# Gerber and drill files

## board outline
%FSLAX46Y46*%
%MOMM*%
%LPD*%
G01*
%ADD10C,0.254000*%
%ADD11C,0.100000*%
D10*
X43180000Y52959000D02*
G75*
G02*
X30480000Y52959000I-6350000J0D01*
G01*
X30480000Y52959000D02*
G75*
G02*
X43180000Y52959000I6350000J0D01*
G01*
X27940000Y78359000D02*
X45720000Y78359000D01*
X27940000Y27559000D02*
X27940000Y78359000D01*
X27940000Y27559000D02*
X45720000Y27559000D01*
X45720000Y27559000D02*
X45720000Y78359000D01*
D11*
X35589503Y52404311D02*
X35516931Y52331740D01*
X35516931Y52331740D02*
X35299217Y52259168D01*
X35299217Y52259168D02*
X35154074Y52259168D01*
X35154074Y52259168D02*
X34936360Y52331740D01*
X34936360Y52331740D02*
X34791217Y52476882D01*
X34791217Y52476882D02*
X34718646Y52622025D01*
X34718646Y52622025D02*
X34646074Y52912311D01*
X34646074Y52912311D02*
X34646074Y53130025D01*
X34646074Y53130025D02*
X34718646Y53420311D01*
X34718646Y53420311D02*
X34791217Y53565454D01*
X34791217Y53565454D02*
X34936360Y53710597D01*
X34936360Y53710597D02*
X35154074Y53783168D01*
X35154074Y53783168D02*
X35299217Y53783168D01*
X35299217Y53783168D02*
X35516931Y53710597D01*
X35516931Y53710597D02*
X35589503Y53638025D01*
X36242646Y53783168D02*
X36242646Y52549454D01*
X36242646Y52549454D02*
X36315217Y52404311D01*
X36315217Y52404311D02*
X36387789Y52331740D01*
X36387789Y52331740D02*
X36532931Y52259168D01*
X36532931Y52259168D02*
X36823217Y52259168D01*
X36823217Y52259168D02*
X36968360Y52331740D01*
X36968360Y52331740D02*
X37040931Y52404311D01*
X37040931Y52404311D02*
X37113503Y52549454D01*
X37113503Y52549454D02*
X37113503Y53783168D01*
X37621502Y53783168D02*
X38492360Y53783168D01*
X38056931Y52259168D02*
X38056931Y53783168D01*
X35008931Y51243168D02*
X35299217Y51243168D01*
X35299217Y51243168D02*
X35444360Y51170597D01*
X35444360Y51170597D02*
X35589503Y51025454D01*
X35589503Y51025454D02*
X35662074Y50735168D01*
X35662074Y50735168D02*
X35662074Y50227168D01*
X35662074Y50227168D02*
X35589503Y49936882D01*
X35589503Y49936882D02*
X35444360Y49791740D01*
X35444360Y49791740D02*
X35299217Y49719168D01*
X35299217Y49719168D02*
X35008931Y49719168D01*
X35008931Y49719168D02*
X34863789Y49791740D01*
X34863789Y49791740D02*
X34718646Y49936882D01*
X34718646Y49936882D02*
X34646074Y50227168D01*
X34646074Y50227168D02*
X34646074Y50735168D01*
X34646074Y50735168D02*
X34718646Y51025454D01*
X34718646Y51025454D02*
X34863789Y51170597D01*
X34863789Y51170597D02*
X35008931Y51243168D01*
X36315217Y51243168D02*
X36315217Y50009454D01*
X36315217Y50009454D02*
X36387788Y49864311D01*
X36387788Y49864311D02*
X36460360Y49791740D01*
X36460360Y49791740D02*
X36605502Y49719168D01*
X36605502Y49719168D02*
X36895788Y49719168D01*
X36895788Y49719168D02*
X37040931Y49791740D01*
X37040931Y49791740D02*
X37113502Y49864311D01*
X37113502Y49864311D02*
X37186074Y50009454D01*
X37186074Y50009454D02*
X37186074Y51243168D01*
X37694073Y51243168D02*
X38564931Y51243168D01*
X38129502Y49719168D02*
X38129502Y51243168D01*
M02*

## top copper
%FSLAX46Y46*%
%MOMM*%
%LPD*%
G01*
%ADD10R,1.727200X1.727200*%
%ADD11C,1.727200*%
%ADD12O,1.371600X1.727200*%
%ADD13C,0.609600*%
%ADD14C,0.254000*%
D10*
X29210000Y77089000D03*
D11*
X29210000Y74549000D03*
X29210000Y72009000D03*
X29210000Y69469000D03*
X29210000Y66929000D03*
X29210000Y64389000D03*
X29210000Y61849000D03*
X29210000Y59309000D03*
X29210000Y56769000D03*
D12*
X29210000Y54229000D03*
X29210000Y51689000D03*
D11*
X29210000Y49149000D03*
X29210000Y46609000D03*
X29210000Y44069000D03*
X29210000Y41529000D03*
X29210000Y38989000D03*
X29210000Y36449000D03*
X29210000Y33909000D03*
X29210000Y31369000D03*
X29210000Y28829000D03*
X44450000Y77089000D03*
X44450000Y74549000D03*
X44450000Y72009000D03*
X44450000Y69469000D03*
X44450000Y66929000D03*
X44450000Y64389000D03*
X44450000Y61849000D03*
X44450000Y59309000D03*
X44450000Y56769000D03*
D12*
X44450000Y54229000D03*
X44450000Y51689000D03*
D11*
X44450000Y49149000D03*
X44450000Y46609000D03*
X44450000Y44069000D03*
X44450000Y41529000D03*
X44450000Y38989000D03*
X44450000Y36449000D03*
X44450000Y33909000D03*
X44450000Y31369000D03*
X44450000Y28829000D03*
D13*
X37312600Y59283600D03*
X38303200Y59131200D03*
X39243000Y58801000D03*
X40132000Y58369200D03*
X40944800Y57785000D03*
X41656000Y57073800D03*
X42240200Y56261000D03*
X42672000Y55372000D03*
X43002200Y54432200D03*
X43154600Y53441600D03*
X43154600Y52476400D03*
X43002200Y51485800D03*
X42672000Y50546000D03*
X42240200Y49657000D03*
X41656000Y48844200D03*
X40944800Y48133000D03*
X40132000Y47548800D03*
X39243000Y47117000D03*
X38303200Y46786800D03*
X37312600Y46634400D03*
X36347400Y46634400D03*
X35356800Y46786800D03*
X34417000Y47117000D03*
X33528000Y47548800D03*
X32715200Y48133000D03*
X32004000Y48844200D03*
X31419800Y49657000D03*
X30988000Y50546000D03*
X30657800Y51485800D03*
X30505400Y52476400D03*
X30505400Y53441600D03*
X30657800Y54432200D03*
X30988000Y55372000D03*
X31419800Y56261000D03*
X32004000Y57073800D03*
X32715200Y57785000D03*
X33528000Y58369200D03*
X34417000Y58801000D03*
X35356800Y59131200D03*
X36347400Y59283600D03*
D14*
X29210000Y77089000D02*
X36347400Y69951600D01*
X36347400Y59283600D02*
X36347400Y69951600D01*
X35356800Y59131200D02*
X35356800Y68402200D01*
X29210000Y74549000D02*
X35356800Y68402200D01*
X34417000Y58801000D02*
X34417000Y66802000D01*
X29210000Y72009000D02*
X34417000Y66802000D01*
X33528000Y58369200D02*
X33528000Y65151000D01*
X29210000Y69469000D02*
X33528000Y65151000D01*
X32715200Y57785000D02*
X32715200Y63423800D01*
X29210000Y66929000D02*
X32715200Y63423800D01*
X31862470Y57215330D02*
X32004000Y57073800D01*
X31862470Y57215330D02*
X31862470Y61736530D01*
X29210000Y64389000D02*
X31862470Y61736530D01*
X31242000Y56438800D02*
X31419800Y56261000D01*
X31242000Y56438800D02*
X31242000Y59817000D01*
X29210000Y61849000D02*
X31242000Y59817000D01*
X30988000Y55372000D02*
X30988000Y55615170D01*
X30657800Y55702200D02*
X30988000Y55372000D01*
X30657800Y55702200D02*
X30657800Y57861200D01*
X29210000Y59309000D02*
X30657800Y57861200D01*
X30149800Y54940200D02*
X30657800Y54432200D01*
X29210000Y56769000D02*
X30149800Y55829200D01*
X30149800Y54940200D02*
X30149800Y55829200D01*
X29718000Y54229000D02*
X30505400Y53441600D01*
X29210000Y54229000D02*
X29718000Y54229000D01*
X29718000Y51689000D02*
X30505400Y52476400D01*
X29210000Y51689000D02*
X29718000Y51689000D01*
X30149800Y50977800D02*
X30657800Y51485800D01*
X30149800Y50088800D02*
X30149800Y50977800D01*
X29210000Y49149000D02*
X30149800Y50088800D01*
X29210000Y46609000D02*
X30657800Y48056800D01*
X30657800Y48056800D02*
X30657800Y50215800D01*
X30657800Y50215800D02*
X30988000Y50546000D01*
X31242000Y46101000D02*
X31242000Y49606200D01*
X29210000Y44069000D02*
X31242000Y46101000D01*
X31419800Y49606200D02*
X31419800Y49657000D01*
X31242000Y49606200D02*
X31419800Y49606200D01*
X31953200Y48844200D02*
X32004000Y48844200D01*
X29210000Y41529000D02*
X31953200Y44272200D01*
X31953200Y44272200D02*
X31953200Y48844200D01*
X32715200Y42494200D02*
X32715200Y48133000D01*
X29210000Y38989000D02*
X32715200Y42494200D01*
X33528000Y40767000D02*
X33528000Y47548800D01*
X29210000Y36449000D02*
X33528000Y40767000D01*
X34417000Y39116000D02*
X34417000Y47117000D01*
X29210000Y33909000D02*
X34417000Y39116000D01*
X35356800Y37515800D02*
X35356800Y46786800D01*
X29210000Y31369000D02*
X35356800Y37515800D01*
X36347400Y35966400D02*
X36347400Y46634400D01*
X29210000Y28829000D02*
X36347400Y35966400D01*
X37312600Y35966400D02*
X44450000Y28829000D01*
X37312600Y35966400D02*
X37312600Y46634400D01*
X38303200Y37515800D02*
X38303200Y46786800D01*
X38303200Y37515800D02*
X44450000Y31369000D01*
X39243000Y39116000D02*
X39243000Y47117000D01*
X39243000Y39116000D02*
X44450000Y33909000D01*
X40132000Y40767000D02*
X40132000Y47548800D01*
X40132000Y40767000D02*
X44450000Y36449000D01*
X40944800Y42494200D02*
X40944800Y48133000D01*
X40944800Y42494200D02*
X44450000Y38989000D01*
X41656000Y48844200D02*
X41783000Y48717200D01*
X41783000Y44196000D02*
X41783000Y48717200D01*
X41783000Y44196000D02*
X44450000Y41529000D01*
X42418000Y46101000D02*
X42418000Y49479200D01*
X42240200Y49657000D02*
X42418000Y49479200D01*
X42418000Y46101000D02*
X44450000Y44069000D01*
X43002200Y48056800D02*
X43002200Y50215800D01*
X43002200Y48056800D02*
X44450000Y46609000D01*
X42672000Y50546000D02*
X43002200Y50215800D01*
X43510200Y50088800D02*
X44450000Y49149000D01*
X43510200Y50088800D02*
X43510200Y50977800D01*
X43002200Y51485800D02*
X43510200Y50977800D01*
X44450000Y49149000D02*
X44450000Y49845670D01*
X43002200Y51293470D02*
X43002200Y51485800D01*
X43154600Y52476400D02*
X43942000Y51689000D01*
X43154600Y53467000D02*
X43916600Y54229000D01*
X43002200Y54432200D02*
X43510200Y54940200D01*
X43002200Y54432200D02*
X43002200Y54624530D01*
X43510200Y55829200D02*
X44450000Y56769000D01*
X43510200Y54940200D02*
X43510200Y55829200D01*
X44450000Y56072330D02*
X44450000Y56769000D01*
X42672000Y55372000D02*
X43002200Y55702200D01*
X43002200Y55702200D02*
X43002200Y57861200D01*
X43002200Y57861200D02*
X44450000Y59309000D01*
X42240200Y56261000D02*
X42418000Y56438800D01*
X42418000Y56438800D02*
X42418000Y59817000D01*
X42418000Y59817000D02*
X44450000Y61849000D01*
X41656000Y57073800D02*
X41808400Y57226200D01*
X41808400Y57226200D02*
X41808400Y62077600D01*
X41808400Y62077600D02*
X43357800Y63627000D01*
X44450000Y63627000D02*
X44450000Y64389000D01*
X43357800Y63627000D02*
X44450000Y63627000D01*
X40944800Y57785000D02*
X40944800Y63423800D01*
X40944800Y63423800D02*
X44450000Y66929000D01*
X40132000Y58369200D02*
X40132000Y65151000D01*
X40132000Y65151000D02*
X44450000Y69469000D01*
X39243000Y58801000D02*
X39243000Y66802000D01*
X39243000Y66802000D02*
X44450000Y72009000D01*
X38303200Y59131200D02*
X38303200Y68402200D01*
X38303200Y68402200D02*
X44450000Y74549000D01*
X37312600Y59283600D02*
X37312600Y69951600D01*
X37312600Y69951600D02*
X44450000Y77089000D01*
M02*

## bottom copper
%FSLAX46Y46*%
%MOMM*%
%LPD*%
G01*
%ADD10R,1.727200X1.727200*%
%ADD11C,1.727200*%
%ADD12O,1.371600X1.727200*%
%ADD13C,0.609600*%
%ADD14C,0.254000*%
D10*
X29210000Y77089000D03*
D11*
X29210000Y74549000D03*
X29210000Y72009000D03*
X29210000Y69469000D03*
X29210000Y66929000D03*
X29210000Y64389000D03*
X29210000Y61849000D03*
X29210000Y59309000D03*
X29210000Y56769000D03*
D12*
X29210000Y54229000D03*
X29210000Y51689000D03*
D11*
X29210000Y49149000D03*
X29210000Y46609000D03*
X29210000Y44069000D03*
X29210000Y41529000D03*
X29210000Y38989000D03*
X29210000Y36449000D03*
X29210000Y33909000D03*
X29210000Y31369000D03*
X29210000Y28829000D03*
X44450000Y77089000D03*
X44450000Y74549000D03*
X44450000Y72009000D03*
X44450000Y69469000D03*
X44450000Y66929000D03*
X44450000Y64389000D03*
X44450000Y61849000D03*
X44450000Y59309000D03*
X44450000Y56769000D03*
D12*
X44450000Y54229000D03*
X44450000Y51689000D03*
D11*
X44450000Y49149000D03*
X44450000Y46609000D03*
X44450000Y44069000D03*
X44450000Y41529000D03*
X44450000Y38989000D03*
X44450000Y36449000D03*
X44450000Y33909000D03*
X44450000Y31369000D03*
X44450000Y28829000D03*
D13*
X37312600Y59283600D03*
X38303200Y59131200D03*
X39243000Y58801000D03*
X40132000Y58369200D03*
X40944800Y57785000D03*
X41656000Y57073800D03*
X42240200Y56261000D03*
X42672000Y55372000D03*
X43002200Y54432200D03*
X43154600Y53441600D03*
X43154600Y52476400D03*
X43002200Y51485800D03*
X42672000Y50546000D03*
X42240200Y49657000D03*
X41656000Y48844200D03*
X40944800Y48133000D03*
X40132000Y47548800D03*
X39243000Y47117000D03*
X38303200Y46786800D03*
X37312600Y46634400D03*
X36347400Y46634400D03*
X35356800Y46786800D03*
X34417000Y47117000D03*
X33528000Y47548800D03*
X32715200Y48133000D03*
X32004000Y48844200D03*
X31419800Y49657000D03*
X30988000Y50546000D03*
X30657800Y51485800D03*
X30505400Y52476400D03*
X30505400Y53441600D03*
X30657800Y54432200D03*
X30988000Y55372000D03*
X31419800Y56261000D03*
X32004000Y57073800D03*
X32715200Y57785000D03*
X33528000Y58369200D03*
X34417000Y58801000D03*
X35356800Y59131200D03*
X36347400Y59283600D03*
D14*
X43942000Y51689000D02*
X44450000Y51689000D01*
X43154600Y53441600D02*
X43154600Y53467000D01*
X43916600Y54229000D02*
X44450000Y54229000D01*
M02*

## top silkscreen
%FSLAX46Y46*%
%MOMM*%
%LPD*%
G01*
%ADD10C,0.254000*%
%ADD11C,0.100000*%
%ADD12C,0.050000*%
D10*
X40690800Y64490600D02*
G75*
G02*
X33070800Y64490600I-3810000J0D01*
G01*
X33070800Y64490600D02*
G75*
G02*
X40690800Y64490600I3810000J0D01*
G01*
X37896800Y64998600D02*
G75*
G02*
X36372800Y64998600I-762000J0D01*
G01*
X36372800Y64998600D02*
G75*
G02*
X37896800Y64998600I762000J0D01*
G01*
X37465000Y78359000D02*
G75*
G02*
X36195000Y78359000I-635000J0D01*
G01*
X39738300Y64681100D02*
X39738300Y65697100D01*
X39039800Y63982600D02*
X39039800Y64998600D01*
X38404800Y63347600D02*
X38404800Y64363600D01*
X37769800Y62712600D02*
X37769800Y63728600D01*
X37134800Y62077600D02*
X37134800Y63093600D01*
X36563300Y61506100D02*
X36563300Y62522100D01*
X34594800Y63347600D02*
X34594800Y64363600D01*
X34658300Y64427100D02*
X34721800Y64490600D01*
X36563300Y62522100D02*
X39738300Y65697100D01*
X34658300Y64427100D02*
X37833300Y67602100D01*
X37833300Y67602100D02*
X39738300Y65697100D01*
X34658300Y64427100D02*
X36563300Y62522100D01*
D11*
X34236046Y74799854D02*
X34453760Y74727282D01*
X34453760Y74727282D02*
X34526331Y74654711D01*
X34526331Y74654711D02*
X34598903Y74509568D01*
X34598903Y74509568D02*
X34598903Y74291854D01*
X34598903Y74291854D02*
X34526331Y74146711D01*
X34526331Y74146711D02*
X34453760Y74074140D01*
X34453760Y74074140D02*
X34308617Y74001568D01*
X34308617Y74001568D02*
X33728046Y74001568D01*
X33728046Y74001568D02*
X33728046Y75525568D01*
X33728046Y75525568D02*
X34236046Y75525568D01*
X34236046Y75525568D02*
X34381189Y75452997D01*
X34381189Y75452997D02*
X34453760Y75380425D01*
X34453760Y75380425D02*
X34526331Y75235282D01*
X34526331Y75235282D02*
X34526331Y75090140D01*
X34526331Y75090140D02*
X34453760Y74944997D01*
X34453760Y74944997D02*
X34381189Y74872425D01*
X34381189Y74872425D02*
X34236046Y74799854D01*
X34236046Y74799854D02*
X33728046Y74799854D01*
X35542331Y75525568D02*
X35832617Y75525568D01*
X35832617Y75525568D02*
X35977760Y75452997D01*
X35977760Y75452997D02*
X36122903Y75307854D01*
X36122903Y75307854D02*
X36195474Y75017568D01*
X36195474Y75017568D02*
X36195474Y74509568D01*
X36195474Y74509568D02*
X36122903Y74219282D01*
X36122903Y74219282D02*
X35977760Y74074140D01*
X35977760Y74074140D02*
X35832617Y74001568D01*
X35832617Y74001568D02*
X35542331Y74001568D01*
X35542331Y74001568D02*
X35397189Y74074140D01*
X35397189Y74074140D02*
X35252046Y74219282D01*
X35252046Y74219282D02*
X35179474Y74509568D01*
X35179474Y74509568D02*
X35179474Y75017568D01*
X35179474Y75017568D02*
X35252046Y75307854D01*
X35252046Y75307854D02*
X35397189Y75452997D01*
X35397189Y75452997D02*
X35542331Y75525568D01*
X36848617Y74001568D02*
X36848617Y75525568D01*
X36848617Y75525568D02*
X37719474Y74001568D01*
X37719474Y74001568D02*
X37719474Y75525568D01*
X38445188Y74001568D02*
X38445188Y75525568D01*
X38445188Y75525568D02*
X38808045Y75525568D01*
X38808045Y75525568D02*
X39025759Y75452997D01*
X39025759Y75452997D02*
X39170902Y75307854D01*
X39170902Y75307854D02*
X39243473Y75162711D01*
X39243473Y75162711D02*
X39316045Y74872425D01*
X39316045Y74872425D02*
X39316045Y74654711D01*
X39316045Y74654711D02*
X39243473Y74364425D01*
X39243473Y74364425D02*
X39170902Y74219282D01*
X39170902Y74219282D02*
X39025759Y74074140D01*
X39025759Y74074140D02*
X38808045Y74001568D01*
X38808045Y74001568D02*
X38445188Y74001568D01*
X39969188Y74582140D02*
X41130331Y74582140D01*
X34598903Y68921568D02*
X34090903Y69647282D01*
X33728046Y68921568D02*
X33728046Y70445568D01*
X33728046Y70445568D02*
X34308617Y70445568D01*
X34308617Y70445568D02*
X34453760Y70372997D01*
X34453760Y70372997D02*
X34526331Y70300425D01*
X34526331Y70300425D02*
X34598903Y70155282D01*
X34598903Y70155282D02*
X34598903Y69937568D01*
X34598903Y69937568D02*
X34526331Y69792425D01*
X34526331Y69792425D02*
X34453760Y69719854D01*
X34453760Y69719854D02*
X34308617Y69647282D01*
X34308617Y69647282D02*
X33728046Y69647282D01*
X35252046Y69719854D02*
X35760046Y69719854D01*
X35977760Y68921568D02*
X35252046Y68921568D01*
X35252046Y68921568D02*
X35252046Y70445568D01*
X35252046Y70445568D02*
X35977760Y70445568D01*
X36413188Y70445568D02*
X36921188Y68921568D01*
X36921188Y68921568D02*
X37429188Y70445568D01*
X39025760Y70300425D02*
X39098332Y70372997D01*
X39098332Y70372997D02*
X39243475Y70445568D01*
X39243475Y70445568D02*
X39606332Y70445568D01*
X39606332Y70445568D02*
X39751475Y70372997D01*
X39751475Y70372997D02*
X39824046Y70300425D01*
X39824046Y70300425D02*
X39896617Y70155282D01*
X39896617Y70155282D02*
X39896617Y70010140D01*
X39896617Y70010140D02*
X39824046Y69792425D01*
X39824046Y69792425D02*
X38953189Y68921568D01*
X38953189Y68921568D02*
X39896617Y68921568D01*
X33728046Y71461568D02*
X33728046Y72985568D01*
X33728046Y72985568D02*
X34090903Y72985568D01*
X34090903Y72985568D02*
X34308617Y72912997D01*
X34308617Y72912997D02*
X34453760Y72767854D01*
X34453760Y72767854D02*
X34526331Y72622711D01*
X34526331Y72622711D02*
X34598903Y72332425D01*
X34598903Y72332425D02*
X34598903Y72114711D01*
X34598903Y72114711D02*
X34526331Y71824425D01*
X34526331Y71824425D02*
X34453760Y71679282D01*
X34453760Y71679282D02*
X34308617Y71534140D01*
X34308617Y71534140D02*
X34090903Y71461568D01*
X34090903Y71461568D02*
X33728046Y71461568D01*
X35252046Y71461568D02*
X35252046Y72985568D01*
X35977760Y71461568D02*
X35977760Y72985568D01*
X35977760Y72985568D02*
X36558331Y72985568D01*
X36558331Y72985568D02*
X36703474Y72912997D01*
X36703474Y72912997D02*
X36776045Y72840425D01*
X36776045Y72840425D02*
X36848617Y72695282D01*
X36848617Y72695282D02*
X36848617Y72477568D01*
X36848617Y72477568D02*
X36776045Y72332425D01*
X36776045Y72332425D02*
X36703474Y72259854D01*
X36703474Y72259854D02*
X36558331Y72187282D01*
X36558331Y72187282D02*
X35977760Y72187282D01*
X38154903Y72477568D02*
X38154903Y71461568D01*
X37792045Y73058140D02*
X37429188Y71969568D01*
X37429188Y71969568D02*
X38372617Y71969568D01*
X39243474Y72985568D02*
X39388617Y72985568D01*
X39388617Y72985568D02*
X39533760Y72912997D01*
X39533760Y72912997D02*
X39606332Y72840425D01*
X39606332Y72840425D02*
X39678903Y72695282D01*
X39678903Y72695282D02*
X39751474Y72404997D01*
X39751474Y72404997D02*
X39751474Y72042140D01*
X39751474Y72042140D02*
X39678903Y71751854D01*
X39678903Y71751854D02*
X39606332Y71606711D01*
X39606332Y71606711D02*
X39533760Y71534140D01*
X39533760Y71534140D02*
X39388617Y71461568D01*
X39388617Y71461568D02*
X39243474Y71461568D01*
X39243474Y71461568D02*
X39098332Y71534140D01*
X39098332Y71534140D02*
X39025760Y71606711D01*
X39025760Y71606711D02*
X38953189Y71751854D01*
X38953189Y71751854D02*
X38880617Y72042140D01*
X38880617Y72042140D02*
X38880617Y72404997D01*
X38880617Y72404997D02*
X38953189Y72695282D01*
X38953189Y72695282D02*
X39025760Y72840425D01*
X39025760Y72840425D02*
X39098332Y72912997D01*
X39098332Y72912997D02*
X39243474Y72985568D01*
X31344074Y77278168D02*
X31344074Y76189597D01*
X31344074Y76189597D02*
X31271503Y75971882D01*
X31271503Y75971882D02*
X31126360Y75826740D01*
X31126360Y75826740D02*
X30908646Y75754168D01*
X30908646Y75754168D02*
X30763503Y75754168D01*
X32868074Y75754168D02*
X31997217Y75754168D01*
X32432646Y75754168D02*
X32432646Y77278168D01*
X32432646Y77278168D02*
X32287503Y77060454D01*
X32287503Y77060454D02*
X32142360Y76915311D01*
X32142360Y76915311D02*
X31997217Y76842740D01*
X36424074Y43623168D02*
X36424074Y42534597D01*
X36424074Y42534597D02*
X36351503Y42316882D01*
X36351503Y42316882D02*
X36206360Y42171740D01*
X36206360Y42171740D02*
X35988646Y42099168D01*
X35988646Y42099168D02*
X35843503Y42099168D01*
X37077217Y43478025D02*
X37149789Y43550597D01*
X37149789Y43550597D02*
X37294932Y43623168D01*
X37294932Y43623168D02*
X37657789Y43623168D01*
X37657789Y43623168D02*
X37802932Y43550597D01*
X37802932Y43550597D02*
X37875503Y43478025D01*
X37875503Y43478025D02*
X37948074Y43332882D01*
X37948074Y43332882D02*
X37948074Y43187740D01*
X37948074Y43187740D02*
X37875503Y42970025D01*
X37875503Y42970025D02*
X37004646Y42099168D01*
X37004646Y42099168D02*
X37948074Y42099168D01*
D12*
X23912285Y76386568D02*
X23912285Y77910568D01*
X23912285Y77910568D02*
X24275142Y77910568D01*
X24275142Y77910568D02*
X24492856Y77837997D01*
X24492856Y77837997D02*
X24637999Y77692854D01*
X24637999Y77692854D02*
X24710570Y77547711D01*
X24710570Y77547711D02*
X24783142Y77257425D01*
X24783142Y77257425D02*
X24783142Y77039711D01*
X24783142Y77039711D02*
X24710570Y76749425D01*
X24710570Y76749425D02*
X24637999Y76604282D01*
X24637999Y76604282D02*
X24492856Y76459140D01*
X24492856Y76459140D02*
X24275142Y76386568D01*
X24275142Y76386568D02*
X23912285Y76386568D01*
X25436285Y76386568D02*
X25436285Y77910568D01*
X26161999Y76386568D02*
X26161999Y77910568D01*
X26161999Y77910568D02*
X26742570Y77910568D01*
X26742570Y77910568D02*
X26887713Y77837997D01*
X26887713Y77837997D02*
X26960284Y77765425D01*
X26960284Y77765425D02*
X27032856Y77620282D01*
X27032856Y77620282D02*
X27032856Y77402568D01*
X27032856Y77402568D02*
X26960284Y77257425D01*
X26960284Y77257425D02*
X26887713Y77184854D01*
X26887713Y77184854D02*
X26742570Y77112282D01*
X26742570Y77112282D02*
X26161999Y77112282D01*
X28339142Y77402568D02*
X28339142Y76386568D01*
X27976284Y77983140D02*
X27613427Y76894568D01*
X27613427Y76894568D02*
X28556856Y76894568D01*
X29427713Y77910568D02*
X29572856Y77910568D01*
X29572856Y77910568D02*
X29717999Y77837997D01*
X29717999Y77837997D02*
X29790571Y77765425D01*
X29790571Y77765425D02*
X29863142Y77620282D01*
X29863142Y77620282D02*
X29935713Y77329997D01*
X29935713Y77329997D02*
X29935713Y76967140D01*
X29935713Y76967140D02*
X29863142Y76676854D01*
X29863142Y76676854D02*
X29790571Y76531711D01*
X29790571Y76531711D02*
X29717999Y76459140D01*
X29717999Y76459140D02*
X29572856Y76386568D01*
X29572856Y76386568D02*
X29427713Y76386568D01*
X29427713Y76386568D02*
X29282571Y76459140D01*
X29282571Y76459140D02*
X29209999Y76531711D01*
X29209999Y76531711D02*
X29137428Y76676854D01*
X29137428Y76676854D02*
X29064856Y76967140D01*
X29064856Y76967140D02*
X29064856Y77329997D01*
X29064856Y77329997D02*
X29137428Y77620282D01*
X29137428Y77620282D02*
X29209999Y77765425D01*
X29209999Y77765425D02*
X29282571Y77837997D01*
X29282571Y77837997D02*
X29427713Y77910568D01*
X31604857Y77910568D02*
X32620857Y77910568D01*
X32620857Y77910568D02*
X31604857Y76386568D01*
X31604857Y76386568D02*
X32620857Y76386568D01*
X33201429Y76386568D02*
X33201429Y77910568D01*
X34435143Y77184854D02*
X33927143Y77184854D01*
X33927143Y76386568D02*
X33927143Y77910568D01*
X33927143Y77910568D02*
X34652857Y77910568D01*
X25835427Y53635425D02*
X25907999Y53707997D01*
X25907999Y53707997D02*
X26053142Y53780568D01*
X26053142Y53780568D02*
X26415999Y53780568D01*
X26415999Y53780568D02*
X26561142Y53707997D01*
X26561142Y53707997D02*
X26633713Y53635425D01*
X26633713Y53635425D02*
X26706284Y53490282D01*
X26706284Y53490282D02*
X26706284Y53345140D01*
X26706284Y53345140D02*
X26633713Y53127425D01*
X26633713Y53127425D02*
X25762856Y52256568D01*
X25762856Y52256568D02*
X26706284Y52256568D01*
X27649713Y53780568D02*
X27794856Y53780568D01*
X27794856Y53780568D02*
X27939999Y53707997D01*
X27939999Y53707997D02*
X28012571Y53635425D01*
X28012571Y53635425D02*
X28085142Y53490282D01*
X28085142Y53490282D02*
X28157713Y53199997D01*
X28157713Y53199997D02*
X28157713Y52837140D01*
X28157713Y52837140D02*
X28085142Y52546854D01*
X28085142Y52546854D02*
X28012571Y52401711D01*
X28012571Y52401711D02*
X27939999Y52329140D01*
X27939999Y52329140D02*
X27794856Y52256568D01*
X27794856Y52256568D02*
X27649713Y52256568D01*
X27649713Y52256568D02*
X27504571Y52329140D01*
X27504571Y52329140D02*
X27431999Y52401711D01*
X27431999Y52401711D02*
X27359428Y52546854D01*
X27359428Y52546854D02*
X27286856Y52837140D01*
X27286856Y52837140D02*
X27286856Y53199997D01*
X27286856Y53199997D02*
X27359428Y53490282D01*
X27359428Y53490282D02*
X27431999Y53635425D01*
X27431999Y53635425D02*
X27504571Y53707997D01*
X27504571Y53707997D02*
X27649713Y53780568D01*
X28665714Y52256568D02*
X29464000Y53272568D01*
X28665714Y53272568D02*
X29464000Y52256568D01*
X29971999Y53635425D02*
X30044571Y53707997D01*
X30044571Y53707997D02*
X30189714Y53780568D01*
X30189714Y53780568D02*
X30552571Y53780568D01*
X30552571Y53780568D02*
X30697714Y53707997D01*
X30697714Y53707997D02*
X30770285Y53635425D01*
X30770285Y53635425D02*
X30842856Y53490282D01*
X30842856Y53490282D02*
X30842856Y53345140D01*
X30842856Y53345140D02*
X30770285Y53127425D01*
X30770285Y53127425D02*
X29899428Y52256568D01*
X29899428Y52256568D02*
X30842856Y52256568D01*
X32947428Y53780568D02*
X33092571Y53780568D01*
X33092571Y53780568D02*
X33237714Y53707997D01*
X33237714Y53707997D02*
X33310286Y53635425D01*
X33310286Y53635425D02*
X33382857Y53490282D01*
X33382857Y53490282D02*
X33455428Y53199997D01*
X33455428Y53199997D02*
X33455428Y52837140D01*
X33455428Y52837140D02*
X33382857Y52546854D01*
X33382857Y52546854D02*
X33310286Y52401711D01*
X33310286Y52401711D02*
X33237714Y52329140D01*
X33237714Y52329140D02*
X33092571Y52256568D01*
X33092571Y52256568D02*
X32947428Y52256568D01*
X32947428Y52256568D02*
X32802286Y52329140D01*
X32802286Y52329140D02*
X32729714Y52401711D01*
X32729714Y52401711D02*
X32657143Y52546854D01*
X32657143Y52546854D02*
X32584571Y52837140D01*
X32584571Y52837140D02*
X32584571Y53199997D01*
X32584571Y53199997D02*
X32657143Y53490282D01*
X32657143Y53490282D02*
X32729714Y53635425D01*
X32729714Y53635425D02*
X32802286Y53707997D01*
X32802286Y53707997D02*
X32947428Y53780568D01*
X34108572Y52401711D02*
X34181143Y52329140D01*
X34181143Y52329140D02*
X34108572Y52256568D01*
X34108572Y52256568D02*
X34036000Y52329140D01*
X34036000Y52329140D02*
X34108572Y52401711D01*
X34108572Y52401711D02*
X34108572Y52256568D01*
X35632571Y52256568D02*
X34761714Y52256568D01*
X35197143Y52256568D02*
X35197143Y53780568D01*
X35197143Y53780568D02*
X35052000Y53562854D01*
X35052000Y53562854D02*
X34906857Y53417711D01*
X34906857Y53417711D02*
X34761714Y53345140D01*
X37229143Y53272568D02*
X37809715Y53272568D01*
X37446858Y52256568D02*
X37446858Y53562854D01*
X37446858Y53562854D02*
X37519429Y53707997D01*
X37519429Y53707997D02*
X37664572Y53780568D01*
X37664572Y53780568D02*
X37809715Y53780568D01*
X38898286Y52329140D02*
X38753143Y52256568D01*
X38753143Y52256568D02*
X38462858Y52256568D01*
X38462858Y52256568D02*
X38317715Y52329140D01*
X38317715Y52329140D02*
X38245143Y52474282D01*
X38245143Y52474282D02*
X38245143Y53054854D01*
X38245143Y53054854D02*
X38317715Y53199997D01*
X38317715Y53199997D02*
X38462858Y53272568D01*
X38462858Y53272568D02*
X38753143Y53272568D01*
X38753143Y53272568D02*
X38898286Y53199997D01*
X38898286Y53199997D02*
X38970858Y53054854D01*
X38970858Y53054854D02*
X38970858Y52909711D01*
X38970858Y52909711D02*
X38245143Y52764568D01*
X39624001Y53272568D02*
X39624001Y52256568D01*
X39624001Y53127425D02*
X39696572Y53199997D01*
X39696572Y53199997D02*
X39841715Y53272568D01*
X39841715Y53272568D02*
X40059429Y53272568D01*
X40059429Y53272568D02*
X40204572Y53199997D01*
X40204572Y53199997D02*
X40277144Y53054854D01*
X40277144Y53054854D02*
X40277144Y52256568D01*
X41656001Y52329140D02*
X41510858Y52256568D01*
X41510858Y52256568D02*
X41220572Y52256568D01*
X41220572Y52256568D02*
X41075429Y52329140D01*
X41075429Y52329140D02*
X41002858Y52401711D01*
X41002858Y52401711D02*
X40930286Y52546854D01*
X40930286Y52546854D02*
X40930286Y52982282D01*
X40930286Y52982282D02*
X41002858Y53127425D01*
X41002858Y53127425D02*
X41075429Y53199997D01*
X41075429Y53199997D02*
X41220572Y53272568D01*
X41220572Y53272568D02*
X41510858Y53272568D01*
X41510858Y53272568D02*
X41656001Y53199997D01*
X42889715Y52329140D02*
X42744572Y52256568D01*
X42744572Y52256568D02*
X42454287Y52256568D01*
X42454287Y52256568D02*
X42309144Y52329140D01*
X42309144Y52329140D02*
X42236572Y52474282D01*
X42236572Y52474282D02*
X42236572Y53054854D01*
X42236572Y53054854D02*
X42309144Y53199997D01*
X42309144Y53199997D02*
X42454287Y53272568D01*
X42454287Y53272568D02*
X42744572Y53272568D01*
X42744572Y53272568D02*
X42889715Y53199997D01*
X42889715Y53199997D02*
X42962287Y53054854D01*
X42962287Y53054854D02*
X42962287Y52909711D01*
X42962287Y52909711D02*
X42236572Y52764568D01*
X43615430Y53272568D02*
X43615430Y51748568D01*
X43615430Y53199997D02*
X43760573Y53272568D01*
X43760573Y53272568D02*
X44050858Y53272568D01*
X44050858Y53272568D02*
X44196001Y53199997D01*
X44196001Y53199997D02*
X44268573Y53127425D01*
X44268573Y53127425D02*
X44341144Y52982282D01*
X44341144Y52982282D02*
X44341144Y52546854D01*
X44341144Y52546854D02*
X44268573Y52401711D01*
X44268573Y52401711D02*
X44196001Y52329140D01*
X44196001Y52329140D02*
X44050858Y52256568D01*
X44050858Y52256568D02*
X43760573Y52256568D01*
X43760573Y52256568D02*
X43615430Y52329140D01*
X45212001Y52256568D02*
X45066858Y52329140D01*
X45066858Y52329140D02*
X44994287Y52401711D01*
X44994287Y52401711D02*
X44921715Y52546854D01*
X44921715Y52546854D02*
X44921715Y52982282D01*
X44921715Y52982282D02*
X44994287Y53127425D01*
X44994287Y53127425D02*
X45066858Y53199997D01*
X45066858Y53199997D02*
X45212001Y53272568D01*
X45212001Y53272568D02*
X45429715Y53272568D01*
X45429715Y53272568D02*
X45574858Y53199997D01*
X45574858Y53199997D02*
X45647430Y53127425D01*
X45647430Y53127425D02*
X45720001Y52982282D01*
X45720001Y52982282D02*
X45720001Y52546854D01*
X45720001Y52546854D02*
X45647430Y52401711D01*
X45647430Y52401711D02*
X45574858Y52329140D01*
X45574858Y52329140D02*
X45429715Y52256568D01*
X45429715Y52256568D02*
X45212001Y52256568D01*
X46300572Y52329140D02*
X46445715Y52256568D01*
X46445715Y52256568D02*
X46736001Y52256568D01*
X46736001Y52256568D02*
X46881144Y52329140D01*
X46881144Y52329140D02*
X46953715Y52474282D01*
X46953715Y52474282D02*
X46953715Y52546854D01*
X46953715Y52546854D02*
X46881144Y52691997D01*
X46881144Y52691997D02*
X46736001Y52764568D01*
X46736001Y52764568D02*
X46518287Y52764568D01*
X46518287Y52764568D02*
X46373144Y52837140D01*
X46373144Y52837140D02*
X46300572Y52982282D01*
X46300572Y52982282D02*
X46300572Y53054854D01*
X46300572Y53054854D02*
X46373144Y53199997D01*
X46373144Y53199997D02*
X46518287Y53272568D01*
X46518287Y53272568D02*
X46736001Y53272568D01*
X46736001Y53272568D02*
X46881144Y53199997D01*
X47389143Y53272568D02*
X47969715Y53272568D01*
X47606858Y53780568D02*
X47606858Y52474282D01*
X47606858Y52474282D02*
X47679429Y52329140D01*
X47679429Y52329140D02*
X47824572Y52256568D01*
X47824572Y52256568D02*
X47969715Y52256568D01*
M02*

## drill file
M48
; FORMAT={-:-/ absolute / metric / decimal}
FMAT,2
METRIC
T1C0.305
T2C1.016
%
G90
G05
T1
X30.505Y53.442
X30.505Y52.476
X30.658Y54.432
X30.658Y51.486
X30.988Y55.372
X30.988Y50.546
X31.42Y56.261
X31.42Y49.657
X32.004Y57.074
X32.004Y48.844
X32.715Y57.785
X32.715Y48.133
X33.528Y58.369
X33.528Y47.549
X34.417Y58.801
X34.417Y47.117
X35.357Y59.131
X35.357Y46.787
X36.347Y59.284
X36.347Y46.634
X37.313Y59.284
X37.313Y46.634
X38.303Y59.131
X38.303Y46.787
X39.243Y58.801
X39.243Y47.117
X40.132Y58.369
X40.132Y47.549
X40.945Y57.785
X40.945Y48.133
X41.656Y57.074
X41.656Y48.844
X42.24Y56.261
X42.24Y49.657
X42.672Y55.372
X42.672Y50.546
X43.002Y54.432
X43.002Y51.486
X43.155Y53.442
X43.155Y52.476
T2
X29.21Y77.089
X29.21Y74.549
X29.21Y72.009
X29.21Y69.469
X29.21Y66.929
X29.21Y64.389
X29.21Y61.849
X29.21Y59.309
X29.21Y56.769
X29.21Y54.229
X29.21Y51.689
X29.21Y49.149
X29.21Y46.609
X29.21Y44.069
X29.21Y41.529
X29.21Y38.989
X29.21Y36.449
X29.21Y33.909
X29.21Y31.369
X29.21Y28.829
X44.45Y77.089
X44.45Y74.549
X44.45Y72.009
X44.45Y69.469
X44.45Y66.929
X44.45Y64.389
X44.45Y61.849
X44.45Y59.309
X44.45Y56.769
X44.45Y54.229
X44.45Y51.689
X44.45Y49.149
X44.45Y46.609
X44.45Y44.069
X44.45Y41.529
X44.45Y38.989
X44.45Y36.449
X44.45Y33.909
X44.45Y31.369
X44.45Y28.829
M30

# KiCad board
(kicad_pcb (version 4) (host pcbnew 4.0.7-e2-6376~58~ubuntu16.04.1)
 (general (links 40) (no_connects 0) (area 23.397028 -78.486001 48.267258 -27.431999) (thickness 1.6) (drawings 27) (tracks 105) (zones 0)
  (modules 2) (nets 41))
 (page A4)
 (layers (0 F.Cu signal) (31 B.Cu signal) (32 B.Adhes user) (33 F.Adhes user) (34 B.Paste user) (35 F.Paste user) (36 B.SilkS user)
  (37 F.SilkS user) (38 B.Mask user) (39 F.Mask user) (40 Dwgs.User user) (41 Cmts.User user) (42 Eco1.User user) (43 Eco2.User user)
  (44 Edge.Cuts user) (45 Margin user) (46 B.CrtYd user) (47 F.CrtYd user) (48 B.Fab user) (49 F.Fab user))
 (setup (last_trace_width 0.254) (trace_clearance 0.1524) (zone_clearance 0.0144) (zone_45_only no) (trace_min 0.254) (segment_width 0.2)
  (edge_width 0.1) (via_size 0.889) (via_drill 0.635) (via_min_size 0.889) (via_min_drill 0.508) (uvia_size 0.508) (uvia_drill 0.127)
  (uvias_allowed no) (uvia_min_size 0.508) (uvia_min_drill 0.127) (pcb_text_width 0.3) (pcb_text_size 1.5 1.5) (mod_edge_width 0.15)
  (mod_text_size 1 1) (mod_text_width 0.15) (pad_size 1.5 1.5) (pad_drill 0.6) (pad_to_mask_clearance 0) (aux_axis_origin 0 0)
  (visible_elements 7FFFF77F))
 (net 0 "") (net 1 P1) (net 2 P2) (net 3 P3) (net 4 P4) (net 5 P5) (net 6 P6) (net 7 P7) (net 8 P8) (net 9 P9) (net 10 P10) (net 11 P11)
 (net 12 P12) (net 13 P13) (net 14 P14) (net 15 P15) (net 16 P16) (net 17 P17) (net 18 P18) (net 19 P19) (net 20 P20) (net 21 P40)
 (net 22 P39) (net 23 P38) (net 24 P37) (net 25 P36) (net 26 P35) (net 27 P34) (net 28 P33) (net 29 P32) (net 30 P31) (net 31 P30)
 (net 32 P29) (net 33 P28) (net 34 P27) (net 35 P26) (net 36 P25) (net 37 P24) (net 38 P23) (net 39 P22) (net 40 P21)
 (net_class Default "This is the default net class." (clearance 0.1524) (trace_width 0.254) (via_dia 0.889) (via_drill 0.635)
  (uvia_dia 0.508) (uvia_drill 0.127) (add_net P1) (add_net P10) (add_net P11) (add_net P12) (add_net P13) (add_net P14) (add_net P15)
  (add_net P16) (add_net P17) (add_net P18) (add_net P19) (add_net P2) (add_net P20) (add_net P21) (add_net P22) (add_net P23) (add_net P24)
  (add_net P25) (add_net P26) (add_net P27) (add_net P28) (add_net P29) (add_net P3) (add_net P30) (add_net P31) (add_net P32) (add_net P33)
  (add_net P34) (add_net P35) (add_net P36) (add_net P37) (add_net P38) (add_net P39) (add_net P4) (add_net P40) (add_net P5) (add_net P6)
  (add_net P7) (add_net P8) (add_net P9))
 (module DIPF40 (layer F.Cu) (at 29.21 -77.089)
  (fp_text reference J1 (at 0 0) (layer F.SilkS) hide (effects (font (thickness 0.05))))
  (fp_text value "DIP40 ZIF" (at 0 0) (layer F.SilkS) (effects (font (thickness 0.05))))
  (pad 1 thru_hole rect (at 0 0) (size 1.7272 1.7272) (drill 1.016) (layers *.Cu *.Paste *.Mask) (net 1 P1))
  (pad 2 thru_hole circle (at 0 2.54) (size 1.7272 1.7272) (drill 1.016) (layers *.Cu *.Paste *.Mask) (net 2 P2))
  (pad 3 thru_hole circle (at 0 5.08) (size 1.7272 1.7272) (drill 1.016) (layers *.Cu *.Paste *.Mask) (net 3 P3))
  (pad 4 thru_hole circle (at 0 7.62) (size 1.7272 1.7272) (drill 1.016) (layers *.Cu *.Paste *.Mask) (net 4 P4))
  (pad 5 thru_hole circle (at 0 10.16) (size 1.7272 1.7272) (drill 1.016) (layers *.Cu *.Paste *.Mask) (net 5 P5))
  (pad 6 thru_hole circle (at 0 12.7) (size 1.7272 1.7272) (drill 1.016) (layers *.Cu *.Paste *.Mask) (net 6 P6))
  (pad 7 thru_hole circle (at 0 15.24) (size 1.7272 1.7272) (drill 1.016) (layers *.Cu *.Paste *.Mask) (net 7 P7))
  (pad 8 thru_hole circle (at 0 17.78) (size 1.7272 1.7272) (drill 1.016) (layers *.Cu *.Paste *.Mask) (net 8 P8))
  (pad 9 thru_hole circle (at 0 20.32) (size 1.7272 1.7272) (drill 1.016) (layers *.Cu *.Paste *.Mask) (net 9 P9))
  (pad 10 thru_hole oval (at 0 22.86) (size 1.3716 1.7272) (drill 1.016) (layers *.Cu *.Paste *.Mask) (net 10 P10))
  (pad 11 thru_hole oval (at 0 25.4) (size 1.3716 1.7272) (drill 1.016) (layers *.Cu *.Paste *.Mask) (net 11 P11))
  (pad 12 thru_hole circle (at 0 27.94) (size 1.7272 1.7272) (drill 1.016) (layers *.Cu *.Paste *.Mask) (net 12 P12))
  (pad 13 thru_hole circle (at 0 30.48) (size 1.7272 1.7272) (drill 1.016) (layers *.Cu *.Paste *.Mask) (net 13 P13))
  (pad 14 thru_hole circle (at 0 33.02) (size 1.7272 1.7272) (drill 1.016) (layers *.Cu *.Paste *.Mask) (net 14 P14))
  (pad 15 thru_hole circle (at 0 35.56) (size 1.7272 1.7272) (drill 1.016) (layers *.Cu *.Paste *.Mask) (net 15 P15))
  (pad 16 thru_hole circle (at 0 38.1) (size 1.7272 1.7272) (drill 1.016) (layers *.Cu *.Paste *.Mask) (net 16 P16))
  (pad 17 thru_hole circle (at 0 40.64) (size 1.7272 1.7272) (drill 1.016) (layers *.Cu *.Paste *.Mask) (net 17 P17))
  (pad 18 thru_hole circle (at 0 43.18) (size 1.7272 1.7272) (drill 1.016) (layers *.Cu *.Paste *.Mask) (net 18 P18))
  (pad 19 thru_hole circle (at 0 45.72) (size 1.7272 1.7272) (drill 1.016) (layers *.Cu *.Paste *.Mask) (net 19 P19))
  (pad 20 thru_hole circle (at 0 48.26) (size 1.7272 1.7272) (drill 1.016) (layers *.Cu *.Paste *.Mask) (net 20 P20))
  (pad 40 thru_hole circle (at 15.24 0) (size 1.7272 1.7272) (drill 1.016) (layers *.Cu *.Paste *.Mask) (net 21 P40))
  (pad 39 thru_hole circle (at 15.24 2.54) (size 1.7272 1.7272) (drill 1.016) (layers *.Cu *.Paste *.Mask) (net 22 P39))
  (pad 38 thru_hole circle (at 15.24 5.08) (size 1.7272 1.7272) (drill 1.016) (layers *.Cu *.Paste *.Mask) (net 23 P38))
  (pad 37 thru_hole circle (at 15.24 7.62) (size 1.7272 1.7272) (drill 1.016) (layers *.Cu *.Paste *.Mask) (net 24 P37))
  (pad 36 thru_hole circle (at 15.24 10.16) (size 1.7272 1.7272) (drill 1.016) (layers *.Cu *.Paste *.Mask) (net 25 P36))
  (pad 35 thru_hole circle (at 15.24 12.7) (size 1.7272 1.7272) (drill 1.016) (layers *.Cu *.Paste *.Mask) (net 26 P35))
  (pad 34 thru_hole circle (at 15.24 15.24) (size 1.7272 1.7272) (drill 1.016) (layers *.Cu *.Paste *.Mask) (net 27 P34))
  (pad 33 thru_hole circle (at 15.24 17.78) (size 1.7272 1.7272) (drill 1.016) (layers *.Cu *.Paste *.Mask) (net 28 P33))
  (pad 32 thru_hole circle (at 15.24 20.32) (size 1.7272 1.7272) (drill 1.016) (layers *.Cu *.Paste *.Mask) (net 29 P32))
  (pad 31 thru_hole oval (at 15.24 22.86) (size 1.3716 1.7272) (drill 1.016) (layers *.Cu *.Paste *.Mask) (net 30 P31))
  (pad 30 thru_hole oval (at 15.24 25.4) (size 1.3716 1.7272) (drill 1.016) (layers *.Cu *.Paste *.Mask) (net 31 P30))
  (pad 29 thru_hole circle (at 15.24 27.94) (size 1.7272 1.7272) (drill 1.016) (layers *.Cu *.Paste *.Mask) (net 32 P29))
  (pad 28 thru_hole circle (at 15.24 30.48) (size 1.7272 1.7272) (drill 1.016) (layers *.Cu *.Paste *.Mask) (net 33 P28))
  (pad 27 thru_hole circle (at 15.24 33.02) (size 1.7272 1.7272) (drill 1.016) (layers *.Cu *.Paste *.Mask) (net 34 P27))
  (pad 26 thru_hole circle (at 15.24 35.56) (size 1.7272 1.7272) (drill 1.016) (layers *.Cu *.Paste *.Mask) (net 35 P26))
  (pad 25 thru_hole circle (at 15.24 38.1) (size 1.7272 1.7272) (drill 1.016) (layers *.Cu *.Paste *.Mask) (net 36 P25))
  (pad 24 thru_hole circle (at 15.24 40.64) (size 1.7272 1.7272) (drill 1.016) (layers *.Cu *.Paste *.Mask) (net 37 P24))
  (pad 23 thru_hole circle (at 15.24 43.18) (size 1.7272 1.7272) (drill 1.016) (layers *.Cu *.Paste *.Mask) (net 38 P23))
  (pad 22 thru_hole circle (at 15.24 45.72) (size 1.7272 1.7272) (drill 1.016) (layers *.Cu *.Paste *.Mask) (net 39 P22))
  (pad 21 thru_hole circle (at 15.24 48.26) (size 1.7272 1.7272) (drill 1.016) (layers *.Cu *.Paste *.Mask) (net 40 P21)))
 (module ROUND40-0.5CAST (layer F.Cu) (at 36.83 -52.959)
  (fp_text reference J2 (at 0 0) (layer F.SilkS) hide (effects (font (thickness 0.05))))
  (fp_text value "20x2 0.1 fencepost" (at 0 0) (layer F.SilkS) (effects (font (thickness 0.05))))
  (pad 40 thru_hole circle (at 0.4826 -6.3246 355.5) (size 0.6096 0.6096) (drill 0.3048) (layers *.Cu *.Paste *.Mask) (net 21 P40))
  (pad 39 thru_hole circle (at 1.4732 -6.1722 346.5) (size 0.6096 0.6096) (drill 0.3048) (layers *.Cu *.Paste *.Mask) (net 22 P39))
  (pad 38 thru_hole circle (at 2.413 -5.842 337.5) (size 0.6096 0.6096) (drill 0.3048) (layers *.Cu *.Paste *.Mask) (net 23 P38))
  (pad 37 thru_hole circle (at 3.302 -5.4102 328.5) (size 0.6096 0.6096) (drill 0.3048) (layers *.Cu *.Paste *.Mask) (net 24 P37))
  (pad 36 thru_hole circle (at 4.1148 -4.826 319.5) (size 0.6096 0.6096) (drill 0.3048) (layers *.Cu *.Paste *.Mask) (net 25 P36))
  (pad 35 thru_hole circle (at 4.826 -4.1148 310.5) (size 0.6096 0.6096) (drill 0.3048) (layers *.Cu *.Paste *.Mask) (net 26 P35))
  (pad 34 thru_hole circle (at 5.4102 -3.302 301.5) (size 0.6096 0.6096) (drill 0.3048) (layers *.Cu *.Paste *.Mask) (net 27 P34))
  (pad 33 thru_hole circle (at 5.842 -2.413 292.5) (size 0.6096 0.6096) (drill 0.3048) (layers *.Cu *.Paste *.Mask) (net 28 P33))
  (pad 32 thru_hole circle (at 6.1722 -1.4732 283.5) (size 0.6096 0.6096) (drill 0.3048) (layers *.Cu *.Paste *.Mask) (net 29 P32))
  (pad 31 thru_hole circle (at 6.3246 -0.4826 274.5) (size 0.6096 0.6096) (drill 0.3048) (layers *.Cu *.Paste *.Mask) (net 30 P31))
  (pad 30 thru_hole circle (at 6.3246 0.4826 265.5) (size 0.6096 0.6096) (drill 0.3048) (layers *.Cu *.Paste *.Mask) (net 31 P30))
  (pad 29 thru_hole circle (at 6.1722 1.4732 256.5) (size 0.6096 0.6096) (drill 0.3048) (layers *.Cu *.Paste *.Mask) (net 32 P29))
  (pad 28 thru_hole circle (at 5.842 2.413 247.5) (size 0.6096 0.6096) (drill 0.3048) (layers *.Cu *.Paste *.Mask) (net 33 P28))
  (pad 27 thru_hole circle (at 5.4102 3.302 238.5) (size 0.6096 0.6096) (drill 0.3048) (layers *.Cu *.Paste *.Mask) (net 34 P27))
  (pad 26 thru_hole circle (at 4.826 4.1148 229.5) (size 0.6096 0.6096) (drill 0.3048) (layers *.Cu *.Paste *.Mask) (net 35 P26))
  (pad 25 thru_hole circle (at 4.1148 4.826 220.5) (size 0.6096 0.6096) (drill 0.3048) (layers *.Cu *.Paste *.Mask) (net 36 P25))
  (pad 24 thru_hole circle (at 3.302 5.4102 211.5) (size 0.6096 0.6096) (drill 0.3048) (layers *.Cu *.Paste *.Mask) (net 37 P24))
  (pad 23 thru_hole circle (at 2.413 5.842 202.5) (size 0.6096 0.6096) (drill 0.3048) (layers *.Cu *.Paste *.Mask) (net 38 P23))
  (pad 22 thru_hole circle (at 1.4732 6.1722 193.5) (size 0.6096 0.6096) (drill 0.3048) (layers *.Cu *.Paste *.Mask) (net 39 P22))
  (pad 21 thru_hole circle (at 0.4826 6.3246 184.5) (size 0.6096 0.6096) (drill 0.3048) (layers *.Cu *.Paste *.Mask) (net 40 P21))
  (pad 20 thru_hole circle (at -0.4826 6.3246 175.5) (size 0.6096 0.6096) (drill 0.3048) (layers *.Cu *.Paste *.Mask) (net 20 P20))
  (pad 19 thru_hole circle (at -1.4732 6.1722 166.5) (size 0.6096 0.6096) (drill 0.3048) (layers *.Cu *.Paste *.Mask) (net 19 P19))
  (pad 18 thru_hole circle (at -2.413 5.842 157.5) (size 0.6096 0.6096) (drill 0.3048) (layers *.Cu *.Paste *.Mask) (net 18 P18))
  (pad 17 thru_hole circle (at -3.302 5.4102 148.5) (size 0.6096 0.6096) (drill 0.3048) (layers *.Cu *.Paste *.Mask) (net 17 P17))
  (pad 16 thru_hole circle (at -4.1148 4.826 139.5) (size 0.6096 0.6096) (drill 0.3048) (layers *.Cu *.Paste *.Mask) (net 16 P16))
  (pad 15 thru_hole circle (at -4.826 4.1148 130.5) (size 0.6096 0.6096) (drill 0.3048) (layers *.Cu *.Paste *.Mask) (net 15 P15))
  (pad 14 thru_hole circle (at -5.4102 3.302 121.5) (size 0.6096 0.6096) (drill 0.3048) (layers *.Cu *.Paste *.Mask) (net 14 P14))
  (pad 13 thru_hole circle (at -5.842 2.413 112.5) (size 0.6096 0.6096) (drill 0.3048) (layers *.Cu *.Paste *.Mask) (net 13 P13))
  (pad 12 thru_hole circle (at -6.1722 1.4732 103.5) (size 0.6096 0.6096) (drill 0.3048) (layers *.Cu *.Paste *.Mask) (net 12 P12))
  (pad 11 thru_hole circle (at -6.3246 0.4826 94.5) (size 0.6096 0.6096) (drill 0.3048) (layers *.Cu *.Paste *.Mask) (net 11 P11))
  (pad 10 thru_hole circle (at -6.3246 -0.4826 85.5) (size 0.6096 0.6096) (drill 0.3048) (layers *.Cu *.Paste *.Mask) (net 10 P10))
  (pad 9 thru_hole circle (at -6.1722 -1.4732 76.5) (size 0.6096 0.6096) (drill 0.3048) (layers *.Cu *.Paste *.Mask) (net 9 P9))
  (pad 8 thru_hole circle (at -5.842 -2.413 67.5) (size 0.6096 0.6096) (drill 0.3048) (layers *.Cu *.Paste *.Mask) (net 8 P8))
  (pad 7 thru_hole circle (at -5.4102 -3.302 58.5) (size 0.6096 0.6096) (drill 0.3048) (layers *.Cu *.Paste *.Mask) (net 7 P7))
  (pad 6 thru_hole circle (at -4.826 -4.1148 49.5) (size 0.6096 0.6096) (drill 0.3048) (layers *.Cu *.Paste *.Mask) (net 6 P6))
  (pad 5 thru_hole circle (at -4.1148 -4.826 40.5) (size 0.6096 0.6096) (drill 0.3048) (layers *.Cu *.Paste *.Mask) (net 5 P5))
  (pad 4 thru_hole circle (at -3.302 -5.4102 31.5) (size 0.6096 0.6096) (drill 0.3048) (layers *.Cu *.Paste *.Mask) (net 4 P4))
  (pad 3 thru_hole circle (at -2.413 -5.842 22.5) (size 0.6096 0.6096) (drill 0.3048) (layers *.Cu *.Paste *.Mask) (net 3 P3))
  (pad 2 thru_hole circle (at -1.4732 -6.1722 13.5) (size 0.6096 0.6096) (drill 0.3048) (layers *.Cu *.Paste *.Mask) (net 2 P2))
  (pad 1 thru_hole circle (at -0.4826 -6.3246 4.5) (size 0.6096 0.6096) (drill 0.3048) (layers *.Cu *.Paste *.Mask) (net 1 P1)))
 (gr_arc (start 36.83 -52.959) (end 43.18 -52.959) (angle -360) (layer Edge.Cuts) (width 0.254))
 (gr_arc (start 36.8808 -64.4906) (end 40.6908 -64.4906) (angle -360) (layer F.SilkS) (width 0.254))
 (gr_arc (start 37.1348 -64.9986) (end 37.8968 -64.9986) (angle -360) (layer F.SilkS) (width 0.254))
 (gr_arc (start 36.83 -78.359) (end 36.195 -78.359) (angle -180) (layer F.SilkS) (width 0.254))
 (gr_line (start 27.94 -78.359) (end 45.72 -78.359) (layer Edge.Cuts) (width 0.254))
 (gr_line (start 27.94 -27.559) (end 27.94 -78.359) (layer Edge.Cuts) (width 0.254))
 (gr_line (start 27.94 -27.559) (end 45.72 -27.559) (layer Edge.Cuts) (width 0.254))
 (gr_line (start 45.72 -27.559) (end 45.72 -78.359) (layer Edge.Cuts) (width 0.254))
 (gr_line (start 39.7383 -64.6811) (end 39.7383 -65.6971) (layer F.SilkS) (width 0.254))
 (gr_line (start 39.0398 -63.9826) (end 39.0398 -64.9986) (layer F.SilkS) (width 0.254))
 (gr_line (start 38.4048 -63.3476) (end 38.4048 -64.3636) (layer F.SilkS) (width 0.254))
 (gr_line (start 37.7698 -62.7126) (end 37.7698 -63.7286) (layer F.SilkS) (width 0.254))
 (gr_line (start 37.1348 -62.0776) (end 37.1348 -63.0936) (layer F.SilkS) (width 0.254))
 (gr_line (start 36.5633 -61.5061) (end 36.5633 -62.5221) (layer F.SilkS) (width 0.254))
 (gr_line (start 34.5948 -63.3476) (end 34.5948 -64.3636) (layer F.SilkS) (width 0.254))
 (gr_line (start 34.6583 -64.4271) (end 34.7218 -64.4906) (layer F.SilkS) (width 0.254))
 (gr_line (start 36.5633 -62.5221) (end 39.7383 -65.6971) (layer F.SilkS) (width 0.254))
 (gr_line (start 34.6583 -64.4271) (end 37.8333 -67.6021) (layer F.SilkS) (width 0.254))
 (gr_line (start 37.8333 -67.6021) (end 39.7383 -65.6971) (layer F.SilkS) (width 0.254))
 (gr_line (start 34.6583 -64.4271) (end 36.5633 -62.5221) (layer F.SilkS) (width 0.254))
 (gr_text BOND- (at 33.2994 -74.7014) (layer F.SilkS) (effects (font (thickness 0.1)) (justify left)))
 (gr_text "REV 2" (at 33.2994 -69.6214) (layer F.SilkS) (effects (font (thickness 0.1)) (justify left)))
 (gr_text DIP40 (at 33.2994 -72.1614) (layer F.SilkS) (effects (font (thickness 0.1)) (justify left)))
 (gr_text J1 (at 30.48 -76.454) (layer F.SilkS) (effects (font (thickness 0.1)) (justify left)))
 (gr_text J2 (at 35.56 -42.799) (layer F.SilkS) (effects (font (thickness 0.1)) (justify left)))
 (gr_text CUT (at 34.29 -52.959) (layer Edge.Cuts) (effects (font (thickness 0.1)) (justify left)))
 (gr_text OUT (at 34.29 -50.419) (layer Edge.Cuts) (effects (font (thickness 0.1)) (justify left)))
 (segment (start 29.21 -77.089) (end 36.3474 -69.9516) (width 0.254) (layer F.Cu) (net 1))
 (segment (start 36.3474 -59.2836) (end 36.3474 -69.9516) (width 0.254) (layer F.Cu) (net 1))
 (segment (start 35.3568 -59.1312) (end 35.3568 -68.4022) (width 0.254) (layer F.Cu) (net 2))
 (segment (start 29.21 -74.549) (end 35.3568 -68.4022) (width 0.254) (layer F.Cu) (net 2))
 (segment (start 34.417 -58.801) (end 34.417 -66.802) (width 0.254) (layer F.Cu) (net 3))
 (segment (start 29.21 -72.009) (end 34.417 -66.802) (width 0.254) (layer F.Cu) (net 3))
 (segment (start 33.528 -58.3692) (end 33.528 -65.151) (width 0.254) (layer F.Cu) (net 4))
 (segment (start 29.21 -69.469) (end 33.528 -65.151) (width 0.254) (layer F.Cu) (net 4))
 (segment (start 32.7152 -57.785) (end 32.7152 -63.4238) (width 0.254) (layer F.Cu) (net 5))
 (segment (start 29.21 -66.929) (end 32.7152 -63.4238) (width 0.254) (layer F.Cu) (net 5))
 (segment (start 31.86247 -57.21533) (end 32.004 -57.0738) (width 0.254) (layer F.Cu) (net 6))
 (segment (start 31.86247 -57.21533) (end 31.86247 -61.73653) (width 0.254) (layer F.Cu) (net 6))
 (segment (start 29.21 -64.389) (end 31.86247 -61.73653) (width 0.254) (layer F.Cu) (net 6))
 (segment (start 31.242 -56.4388) (end 31.4198 -56.261) (width 0.254) (layer F.Cu) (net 7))
 (segment (start 31.242 -56.4388) (end 31.242 -59.817) (width 0.254) (layer F.Cu) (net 7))
 (segment (start 29.21 -61.849) (end 31.242 -59.817) (width 0.254) (layer F.Cu) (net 7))
 (segment (start 30.988 -55.372) (end 30.988 -55.61517) (width 0.254) (layer F.Cu) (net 8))
 (segment (start 30.6578 -55.7022) (end 30.988 -55.372) (width 0.254) (layer F.Cu) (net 8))
 (segment (start 30.6578 -55.7022) (end 30.6578 -57.8612) (width 0.254) (layer F.Cu) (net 8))
 (segment (start 29.21 -59.309) (end 30.6578 -57.8612) (width 0.254) (layer F.Cu) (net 8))
 (segment (start 30.1498 -54.9402) (end 30.6578 -54.4322) (width 0.254) (layer F.Cu) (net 9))
 (segment (start 29.21 -56.769) (end 30.1498 -55.8292) (width 0.254) (layer F.Cu) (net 9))
 (segment (start 30.1498 -54.9402) (end 30.1498 -55.8292) (width 0.254) (layer F.Cu) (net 9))
 (segment (start 29.718 -54.229) (end 30.5054 -53.4416) (width 0.254) (layer F.Cu) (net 10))
 (segment (start 29.21 -54.229) (end 29.718 -54.229) (width 0.254) (layer F.Cu) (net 10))
 (segment (start 29.718 -51.689) (end 30.5054 -52.4764) (width 0.254) (layer F.Cu) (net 11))
 (segment (start 29.21 -51.689) (end 29.718 -51.689) (width 0.254) (layer F.Cu) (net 11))
 (segment (start 30.1498 -50.9778) (end 30.6578 -51.4858) (width 0.254) (layer F.Cu) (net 12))
 (segment (start 30.1498 -50.0888) (end 30.1498 -50.9778) (width 0.254) (layer F.Cu) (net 12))
 (segment (start 29.21 -49.149) (end 30.1498 -50.0888) (width 0.254) (layer F.Cu) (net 12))
 (segment (start 29.21 -46.609) (end 30.6578 -48.0568) (width 0.254) (layer F.Cu) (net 13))
 (segment (start 30.6578 -48.0568) (end 30.6578 -50.2158) (width 0.254) (layer F.Cu) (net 13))
 (segment (start 30.6578 -50.2158) (end 30.988 -50.546) (width 0.254) (layer F.Cu) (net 13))
 (segment (start 31.242 -46.101) (end 31.242 -49.6062) (width 0.254) (layer F.Cu) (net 14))
 (segment (start 29.21 -44.069) (end 31.242 -46.101) (width 0.254) (layer F.Cu) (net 14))
 (segment (start 31.4198 -49.6062) (end 31.4198 -49.657) (width 0.254) (layer F.Cu) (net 14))
 (segment (start 31.242 -49.6062) (end 31.4198 -49.6062) (width 0.254) (layer F.Cu) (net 14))
 (segment (start 31.9532 -48.8442) (end 32.004 -48.8442) (width 0.254) (layer F.Cu) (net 15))
 (segment (start 29.21 -41.529) (end 31.9532 -44.2722) (width 0.254) (layer F.Cu) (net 15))
 (segment (start 31.9532 -44.2722) (end 31.9532 -48.8442) (width 0.254) (layer F.Cu) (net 15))
 (segment (start 32.7152 -42.4942) (end 32.7152 -48.133) (width 0.254) (layer F.Cu) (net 16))
 (segment (start 29.21 -38.989) (end 32.7152 -42.4942) (width 0.254) (layer F.Cu) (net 16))
 (segment (start 33.528 -40.767) (end 33.528 -47.5488) (width 0.254) (layer F.Cu) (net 17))
 (segment (start 29.21 -36.449) (end 33.528 -40.767) (width 0.254) (layer F.Cu) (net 17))
 (segment (start 34.417 -39.116) (end 34.417 -47.117) (width 0.254) (layer F.Cu) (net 18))
 (segment (start 29.21 -33.909) (end 34.417 -39.116) (width 0.254) (layer F.Cu) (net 18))
 (segment (start 35.3568 -37.5158) (end 35.3568 -46.7868) (width 0.254) (layer F.Cu) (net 19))
 (segment (start 29.21 -31.369) (end 35.3568 -37.5158) (width 0.254) (layer F.Cu) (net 19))
 (segment (start 36.3474 -35.9664) (end 36.3474 -46.6344) (width 0.254) (layer F.Cu) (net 20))
 (segment (start 29.21 -28.829) (end 36.3474 -35.9664) (width 0.254) (layer F.Cu) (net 20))
 (segment (start 37.3126 -35.9664) (end 44.45 -28.829) (width 0.254) (layer F.Cu) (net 40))
 (segment (start 37.3126 -35.9664) (end 37.3126 -46.6344) (width 0.254) (layer F.Cu) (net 40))
 (segment (start 38.3032 -37.5158) (end 38.3032 -46.7868) (width 0.254) (layer F.Cu) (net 39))
 (segment (start 38.3032 -37.5158) (end 44.45 -31.369) (width 0.254) (layer F.Cu) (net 39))
 (segment (start 39.243 -39.116) (end 39.243 -47.117) (width 0.254) (layer F.Cu) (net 38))
 (segment (start 39.243 -39.116) (end 44.45 -33.909) (width 0.254) (layer F.Cu) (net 38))
 (segment (start 40.132 -40.767) (end 40.132 -47.5488) (width 0.254) (layer F.Cu) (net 37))
 (segment (start 40.132 -40.767) (end 44.45 -36.449) (width 0.254) (layer F.Cu) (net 37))
 (segment (start 40.9448 -42.4942) (end 40.9448 -48.133) (width 0.254) (layer F.Cu) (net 36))
 (segment (start 40.9448 -42.4942) (end 44.45 -38.989) (width 0.254) (layer F.Cu) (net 36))
 (segment (start 41.656 -48.8442) (end 41.783 -48.7172) (width 0.254) (layer F.Cu) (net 35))
 (segment (start 41.783 -44.196) (end 41.783 -48.7172) (width 0.254) (layer F.Cu) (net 35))
 (segment (start 41.783 -44.196) (end 44.45 -41.529) (width 0.254) (layer F.Cu) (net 35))
 (segment (start 42.418 -46.101) (end 42.418 -49.4792) (width 0.254) (layer F.Cu) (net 34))
 (segment (start 42.2402 -49.657) (end 42.418 -49.4792) (width 0.254) (layer F.Cu) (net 34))
 (segment (start 42.418 -46.101) (end 44.45 -44.069) (width 0.254) (layer F.Cu) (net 34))
 (segment (start 43.0022 -48.0568) (end 43.0022 -50.2158) (width 0.254) (layer F.Cu) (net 33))
 (segment (start 43.0022 -48.0568) (end 44.45 -46.609) (width 0.254) (layer F.Cu) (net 33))
 (segment (start 42.672 -50.546) (end 43.0022 -50.2158) (width 0.254) (layer F.Cu) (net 33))
 (segment (start 43.5102 -50.0888) (end 44.45 -49.149) (width 0.254) (layer F.Cu) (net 32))
 (segment (start 43.5102 -50.0888) (end 43.5102 -50.9778) (width 0.254) (layer F.Cu) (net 32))
 (segment (start 43.0022 -51.4858) (end 43.5102 -50.9778) (width 0.254) (layer F.Cu) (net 32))
 (segment (start 44.45 -49.149) (end 44.45 -49.84567) (width 0.254) (layer F.Cu) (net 32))
 (segment (start 43.0022 -51.29347) (end 43.0022 -51.4858) (width 0.254) (layer F.Cu) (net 32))
 (segment (start 43.942 -51.689) (end 44.45 -51.689) (width 0.254) (layer B.Cu) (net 31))
 (segment (start 43.1546 -52.4764) (end 43.942 -51.689) (width 0.254) (layer F.Cu) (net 31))
 (segment (start 43.1546 -53.4416) (end 43.1546 -53.467) (width 0.254) (layer B.Cu) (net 30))
 (segment (start 43.9166 -54.229) (end 44.45 -54.229) (width 0.254) (layer B.Cu) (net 30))
 (segment (start 43.1546 -53.467) (end 43.9166 -54.229) (width 0.254) (layer F.Cu) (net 30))
 (segment (start 43.0022 -54.4322) (end 43.5102 -54.9402) (width 0.254) (layer F.Cu) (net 29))
 (segment (start 43.0022 -54.4322) (end 43.0022 -54.62453) (width 0.254) (layer F.Cu) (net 29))
 (segment (start 43.5102 -55.8292) (end 44.45 -56.769) (width 0.254) (layer F.Cu) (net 29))
 (segment (start 43.5102 -54.9402) (end 43.5102 -55.8292) (width 0.254) (layer F.Cu) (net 29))
 (segment (start 44.45 -56.07233) (end 44.45 -56.769) (width 0.254) (layer F.Cu) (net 29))
 (segment (start 42.672 -55.372) (end 43.0022 -55.7022) (width 0.254) (layer F.Cu) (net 28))
 (segment (start 43.0022 -55.7022) (end 43.0022 -57.8612) (width 0.254) (layer F.Cu) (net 28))
 (segment (start 43.0022 -57.8612) (end 44.45 -59.309) (width 0.254) (layer F.Cu) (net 28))
 (segment (start 42.2402 -56.261) (end 42.418 -56.4388) (width 0.254) (layer F.Cu) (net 27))
 (segment (start 42.418 -56.4388) (end 42.418 -59.817) (width 0.254) (layer F.Cu) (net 27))
 (segment (start 42.418 -59.817) (end 44.45 -61.849) (width 0.254) (layer F.Cu) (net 27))
 (segment (start 41.656 -57.0738) (end 41.8084 -57.2262) (width 0.254) (layer F.Cu) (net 26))
 (segment (start 41.8084 -57.2262) (end 41.8084 -62.0776) (width 0.254) (layer F.Cu) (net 26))
 (segment (start 41.8084 -62.0776) (end 43.3578 -63.627) (width 0.254) (layer F.Cu) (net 26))
 (segment (start 44.45 -63.627) (end 44.45 -64.389) (width 0.254) (layer F.Cu) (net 26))
 (segment (start 43.3578 -63.627) (end 44.45 -63.627) (width 0.254) (layer F.Cu) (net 26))
 (segment (start 40.9448 -57.785) (end 40.9448 -63.4238) (width 0.254) (layer F.Cu) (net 25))
 (segment (start 40.9448 -63.4238) (end 44.45 -66.929) (width 0.254) (layer F.Cu) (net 25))
 (segment (start 40.132 -58.3692) (end 40.132 -65.151) (width 0.254) (layer F.Cu) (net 24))
 (segment (start 40.132 -65.151) (end 44.45 -69.469) (width 0.254) (layer F.Cu) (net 24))
 (segment (start 39.243 -58.801) (end 39.243 -66.802) (width 0.254) (layer F.Cu) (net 23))
 (segment (start 39.243 -66.802) (end 44.45 -72.009) (width 0.254) (layer F.Cu) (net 23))
 (segment (start 38.3032 -59.1312) (end 38.3032 -68.4022) (width 0.254) (layer F.Cu) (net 22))
 (segment (start 38.3032 -68.4022) (end 44.45 -74.549) (width 0.254) (layer F.Cu) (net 22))
 (segment (start 37.3126 -59.2836) (end 37.3126 -69.9516) (width 0.254) (layer F.Cu) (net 21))
 (segment (start 37.3126 -69.9516) (end 44.45 -77.089) (width 0.254) (layer F.Cu) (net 21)))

